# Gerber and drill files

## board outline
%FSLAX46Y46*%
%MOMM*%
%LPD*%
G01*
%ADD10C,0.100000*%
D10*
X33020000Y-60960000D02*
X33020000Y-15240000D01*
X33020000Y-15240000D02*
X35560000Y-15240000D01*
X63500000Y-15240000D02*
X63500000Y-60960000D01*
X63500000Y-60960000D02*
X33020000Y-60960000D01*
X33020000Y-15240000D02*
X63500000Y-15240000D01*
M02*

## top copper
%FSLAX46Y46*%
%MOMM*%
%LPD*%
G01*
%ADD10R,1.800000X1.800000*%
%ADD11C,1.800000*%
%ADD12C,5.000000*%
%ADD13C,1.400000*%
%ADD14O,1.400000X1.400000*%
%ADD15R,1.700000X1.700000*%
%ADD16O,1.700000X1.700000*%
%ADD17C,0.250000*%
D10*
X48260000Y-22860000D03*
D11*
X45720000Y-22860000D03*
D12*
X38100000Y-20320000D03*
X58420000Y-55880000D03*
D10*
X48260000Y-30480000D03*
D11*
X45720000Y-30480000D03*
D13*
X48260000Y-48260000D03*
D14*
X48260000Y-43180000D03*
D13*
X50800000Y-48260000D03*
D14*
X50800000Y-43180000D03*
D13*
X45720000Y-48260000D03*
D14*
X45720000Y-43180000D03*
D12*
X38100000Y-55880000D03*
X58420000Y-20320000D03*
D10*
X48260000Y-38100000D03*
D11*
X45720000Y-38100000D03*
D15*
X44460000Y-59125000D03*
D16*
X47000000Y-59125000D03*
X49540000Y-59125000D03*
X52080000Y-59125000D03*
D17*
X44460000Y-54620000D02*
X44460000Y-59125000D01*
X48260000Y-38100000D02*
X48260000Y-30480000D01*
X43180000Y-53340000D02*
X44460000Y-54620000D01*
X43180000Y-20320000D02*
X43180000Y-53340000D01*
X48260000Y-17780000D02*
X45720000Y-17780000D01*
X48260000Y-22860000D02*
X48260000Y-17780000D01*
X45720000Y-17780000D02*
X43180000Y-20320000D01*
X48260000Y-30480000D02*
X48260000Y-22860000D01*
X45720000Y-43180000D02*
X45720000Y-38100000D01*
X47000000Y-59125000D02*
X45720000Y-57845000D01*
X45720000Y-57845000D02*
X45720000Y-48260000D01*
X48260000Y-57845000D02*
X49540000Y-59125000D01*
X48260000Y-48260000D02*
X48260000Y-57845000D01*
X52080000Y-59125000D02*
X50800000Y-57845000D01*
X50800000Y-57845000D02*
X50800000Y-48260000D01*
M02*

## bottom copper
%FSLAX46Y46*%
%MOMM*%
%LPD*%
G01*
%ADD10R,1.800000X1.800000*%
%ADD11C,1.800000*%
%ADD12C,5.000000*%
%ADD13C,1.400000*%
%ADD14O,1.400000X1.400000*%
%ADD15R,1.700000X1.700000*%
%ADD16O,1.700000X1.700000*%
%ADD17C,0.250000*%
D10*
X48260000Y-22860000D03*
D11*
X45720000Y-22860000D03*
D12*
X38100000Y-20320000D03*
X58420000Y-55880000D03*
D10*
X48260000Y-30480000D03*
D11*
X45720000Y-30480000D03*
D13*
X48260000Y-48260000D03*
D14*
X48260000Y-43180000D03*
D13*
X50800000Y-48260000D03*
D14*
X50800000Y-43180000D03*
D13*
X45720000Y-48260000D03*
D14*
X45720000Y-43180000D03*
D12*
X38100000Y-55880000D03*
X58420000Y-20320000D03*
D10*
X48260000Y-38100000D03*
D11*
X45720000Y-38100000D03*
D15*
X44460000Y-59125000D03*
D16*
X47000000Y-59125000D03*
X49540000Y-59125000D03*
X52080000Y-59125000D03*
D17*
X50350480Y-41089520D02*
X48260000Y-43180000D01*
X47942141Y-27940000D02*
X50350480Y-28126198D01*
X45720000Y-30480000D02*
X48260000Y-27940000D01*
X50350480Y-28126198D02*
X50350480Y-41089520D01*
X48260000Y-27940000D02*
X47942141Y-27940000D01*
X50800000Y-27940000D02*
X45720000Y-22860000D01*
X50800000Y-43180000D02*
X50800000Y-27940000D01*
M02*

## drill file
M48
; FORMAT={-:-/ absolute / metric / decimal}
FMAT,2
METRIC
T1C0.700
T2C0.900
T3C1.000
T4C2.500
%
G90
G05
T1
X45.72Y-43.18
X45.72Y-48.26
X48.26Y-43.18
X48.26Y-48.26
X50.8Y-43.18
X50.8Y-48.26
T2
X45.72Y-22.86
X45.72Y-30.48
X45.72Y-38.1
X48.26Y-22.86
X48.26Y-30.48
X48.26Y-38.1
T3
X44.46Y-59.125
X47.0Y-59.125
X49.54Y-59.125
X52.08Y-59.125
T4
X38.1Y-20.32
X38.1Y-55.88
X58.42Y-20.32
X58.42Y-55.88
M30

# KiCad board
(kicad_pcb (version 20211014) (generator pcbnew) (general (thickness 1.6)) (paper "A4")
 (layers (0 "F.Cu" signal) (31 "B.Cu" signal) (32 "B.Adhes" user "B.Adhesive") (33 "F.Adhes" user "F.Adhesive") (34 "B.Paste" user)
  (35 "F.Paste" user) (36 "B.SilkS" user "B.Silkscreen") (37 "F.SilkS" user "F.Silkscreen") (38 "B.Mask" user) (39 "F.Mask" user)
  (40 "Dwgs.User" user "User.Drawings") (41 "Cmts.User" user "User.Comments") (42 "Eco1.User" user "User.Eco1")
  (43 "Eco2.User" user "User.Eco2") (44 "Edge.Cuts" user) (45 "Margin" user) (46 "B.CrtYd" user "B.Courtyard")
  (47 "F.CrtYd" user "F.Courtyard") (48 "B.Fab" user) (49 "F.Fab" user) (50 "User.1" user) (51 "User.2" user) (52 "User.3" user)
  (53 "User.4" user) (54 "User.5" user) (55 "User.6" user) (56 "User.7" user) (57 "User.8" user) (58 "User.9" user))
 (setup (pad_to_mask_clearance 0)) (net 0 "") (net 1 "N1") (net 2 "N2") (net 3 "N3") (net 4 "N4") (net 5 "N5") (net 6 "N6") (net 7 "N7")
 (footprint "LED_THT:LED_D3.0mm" (layer "F.Cu") (at 48.26 22.86 180)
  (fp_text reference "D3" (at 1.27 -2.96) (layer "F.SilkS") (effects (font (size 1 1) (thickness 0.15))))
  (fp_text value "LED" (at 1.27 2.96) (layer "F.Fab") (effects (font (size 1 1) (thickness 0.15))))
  (pad "1" thru_hole rect (at 0 0 180) (size 1.8 1.8) (drill 0.9) (layers *.Cu *.Mask) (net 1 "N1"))
  (pad "2" thru_hole circle (at 2.54 0 180) (size 1.8 1.8) (drill 0.9) (layers *.Cu *.Mask) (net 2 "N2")))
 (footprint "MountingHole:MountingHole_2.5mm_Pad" (layer "F.Cu") (at 38.1 20.32)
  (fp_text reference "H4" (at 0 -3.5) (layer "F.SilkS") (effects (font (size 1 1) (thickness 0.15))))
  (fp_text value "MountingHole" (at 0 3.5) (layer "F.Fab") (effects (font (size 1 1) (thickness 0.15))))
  (pad "1" thru_hole circle (at 0 0) (size 5 5) (drill 2.5) (layers *.Cu *.Mask)))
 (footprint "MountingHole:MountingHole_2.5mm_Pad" (layer "F.Cu") (at 58.42 55.88)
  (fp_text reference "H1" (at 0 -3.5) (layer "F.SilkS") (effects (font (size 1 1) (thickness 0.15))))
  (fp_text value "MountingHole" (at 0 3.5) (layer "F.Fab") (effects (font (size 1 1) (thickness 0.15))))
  (pad "1" thru_hole circle (at 0 0) (size 5 5) (drill 2.5) (layers *.Cu *.Mask)))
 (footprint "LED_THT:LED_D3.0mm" (layer "F.Cu") (at 48.26 30.48 180)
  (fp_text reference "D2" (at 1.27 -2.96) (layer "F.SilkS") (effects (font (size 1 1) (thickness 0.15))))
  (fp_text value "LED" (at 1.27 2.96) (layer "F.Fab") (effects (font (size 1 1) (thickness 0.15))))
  (pad "1" thru_hole rect (at 0 0 180) (size 1.8 1.8) (drill 0.9) (layers *.Cu *.Mask) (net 1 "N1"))
  (pad "2" thru_hole circle (at 2.54 0 180) (size 1.8 1.8) (drill 0.9) (layers *.Cu *.Mask) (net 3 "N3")))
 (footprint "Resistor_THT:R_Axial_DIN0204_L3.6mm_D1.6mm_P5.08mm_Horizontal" (layer "F.Cu") (at 48.26 48.26 90)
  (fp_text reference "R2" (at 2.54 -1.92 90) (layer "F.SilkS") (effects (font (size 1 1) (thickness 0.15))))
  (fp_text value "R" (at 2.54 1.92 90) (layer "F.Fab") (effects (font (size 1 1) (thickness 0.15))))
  (pad "1" thru_hole circle (at 0 0 90) (size 1.4 1.4) (drill 0.7) (layers *.Cu *.Mask) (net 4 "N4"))
  (pad "2" thru_hole oval (at 5.08 0 90) (size 1.4 1.4) (drill 0.7) (layers *.Cu *.Mask) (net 3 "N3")))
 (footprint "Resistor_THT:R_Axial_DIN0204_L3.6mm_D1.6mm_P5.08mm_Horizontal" (layer "F.Cu") (at 50.8 48.26 90)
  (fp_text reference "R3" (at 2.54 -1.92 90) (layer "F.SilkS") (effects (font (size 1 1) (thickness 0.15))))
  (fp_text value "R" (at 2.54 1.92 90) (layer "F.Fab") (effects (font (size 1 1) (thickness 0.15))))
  (pad "1" thru_hole circle (at 0 0 90) (size 1.4 1.4) (drill 0.7) (layers *.Cu *.Mask) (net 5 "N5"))
  (pad "2" thru_hole oval (at 5.08 0 90) (size 1.4 1.4) (drill 0.7) (layers *.Cu *.Mask) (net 2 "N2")))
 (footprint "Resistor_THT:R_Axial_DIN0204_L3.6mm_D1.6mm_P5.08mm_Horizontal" (layer "F.Cu") (at 45.72 48.26 90)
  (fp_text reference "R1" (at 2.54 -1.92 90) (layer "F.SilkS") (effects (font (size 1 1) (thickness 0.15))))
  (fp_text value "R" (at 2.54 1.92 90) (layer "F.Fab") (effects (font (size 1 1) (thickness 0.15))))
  (pad "1" thru_hole circle (at 0 0 90) (size 1.4 1.4) (drill 0.7) (layers *.Cu *.Mask) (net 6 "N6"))
  (pad "2" thru_hole oval (at 5.08 0 90) (size 1.4 1.4) (drill 0.7) (layers *.Cu *.Mask) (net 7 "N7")))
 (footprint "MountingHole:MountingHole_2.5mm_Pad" (layer "F.Cu") (at 38.1 55.88)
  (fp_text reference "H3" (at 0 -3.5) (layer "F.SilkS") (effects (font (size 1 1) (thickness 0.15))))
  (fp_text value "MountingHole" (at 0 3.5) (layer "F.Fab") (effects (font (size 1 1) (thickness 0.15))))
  (pad "1" thru_hole circle (at 0 0) (size 5 5) (drill 2.5) (layers *.Cu *.Mask)))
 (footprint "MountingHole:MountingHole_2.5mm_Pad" (layer "F.Cu") (at 58.42 20.32)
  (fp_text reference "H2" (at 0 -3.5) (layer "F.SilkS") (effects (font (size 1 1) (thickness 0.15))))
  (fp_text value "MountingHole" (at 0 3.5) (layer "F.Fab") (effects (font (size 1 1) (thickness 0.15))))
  (pad "1" thru_hole circle (at 0 0) (size 5 5) (drill 2.5) (layers *.Cu *.Mask)))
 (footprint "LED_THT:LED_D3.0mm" (layer "F.Cu") (at 48.26 38.1 180)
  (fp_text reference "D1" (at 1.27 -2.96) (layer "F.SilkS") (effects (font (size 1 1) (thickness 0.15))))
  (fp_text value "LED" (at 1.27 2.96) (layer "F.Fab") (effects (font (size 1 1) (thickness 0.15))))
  (pad "1" thru_hole rect (at 0 0 180) (size 1.8 1.8) (drill 0.9) (layers *.Cu *.Mask) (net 1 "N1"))
  (pad "2" thru_hole circle (at 2.54 0 180) (size 1.8 1.8) (drill 0.9) (layers *.Cu *.Mask) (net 7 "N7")))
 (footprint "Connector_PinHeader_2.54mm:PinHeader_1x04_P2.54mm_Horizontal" (layer "B.Cu") (at 44.46 59.125 -90)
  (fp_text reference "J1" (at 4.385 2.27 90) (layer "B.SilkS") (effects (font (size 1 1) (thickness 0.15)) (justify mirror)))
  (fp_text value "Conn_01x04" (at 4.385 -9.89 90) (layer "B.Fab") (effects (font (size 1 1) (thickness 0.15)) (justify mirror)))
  (pad "1" thru_hole rect (at 0 0 270) (size 1.7 1.7) (drill 1) (layers *.Cu *.Mask) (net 1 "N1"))
  (pad "2" thru_hole oval (at 0 -2.54 270) (size 1.7 1.7) (drill 1) (layers *.Cu *.Mask) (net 6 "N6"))
  (pad "3" thru_hole oval (at 0 -5.08 270) (size 1.7 1.7) (drill 1) (layers *.Cu *.Mask) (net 4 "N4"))
  (pad "4" thru_hole oval (at 0 -7.62 270) (size 1.7 1.7) (drill 1) (layers *.Cu *.Mask) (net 5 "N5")))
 (gr_line (start 33.02 60.96) (end 33.02 15.24) (layer "Edge.Cuts") (width 0.1))
 (gr_line (start 33.02 15.24) (end 35.56 15.24) (layer "Edge.Cuts") (width 0.1))
 (gr_line (start 63.5 15.24) (end 63.5 60.96) (layer "Edge.Cuts") (width 0.1))
 (gr_line (start 63.5 60.96) (end 33.02 60.96) (layer "Edge.Cuts") (width 0.1))
 (gr_line (start 33.02 15.24) (end 63.5 15.24) (layer "Edge.Cuts") (width 0.1))
 (segment (start 44.46 54.62) (end 44.46 59.125) (width 0.25) (layer "F.Cu") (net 1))
 (segment (start 48.26 38.1) (end 48.26 30.48) (width 0.25) (layer "F.Cu") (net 1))
 (segment (start 43.18 53.34) (end 44.46 54.62) (width 0.25) (layer "F.Cu") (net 1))
 (segment (start 43.18 20.32) (end 43.18 53.34) (width 0.25) (layer "F.Cu") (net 1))
 (segment (start 48.26 17.78) (end 45.72 17.78) (width 0.25) (layer "F.Cu") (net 1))
 (segment (start 48.26 22.86) (end 48.26 17.78) (width 0.25) (layer "F.Cu") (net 1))
 (segment (start 45.72 17.78) (end 43.18 20.32) (width 0.25) (layer "F.Cu") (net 1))
 (segment (start 48.26 30.48) (end 48.26 22.86) (width 0.25) (layer "F.Cu") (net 1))
 (segment (start 45.72 43.18) (end 45.72 38.1) (width 0.25) (layer "F.Cu") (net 7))
 (segment (start 50.35048 41.08952) (end 48.26 43.18) (width 0.25) (layer "B.Cu") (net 3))
 (segment (start 47.942141 27.94) (end 50.35048 28.126198) (width 0.25) (layer "B.Cu") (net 3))
 (segment (start 45.72 30.48) (end 48.26 27.94) (width 0.25) (layer "B.Cu") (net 3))
 (segment (start 50.35048 28.126198) (end 50.35048 41.08952) (width 0.25) (layer "B.Cu") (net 3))
 (segment (start 48.26 27.94) (end 47.942141 27.94) (width 0.25) (layer "B.Cu") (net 3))
 (segment (start 50.8 27.94) (end 45.72 22.86) (width 0.25) (layer "B.Cu") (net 2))
 (segment (start 50.8 43.18) (end 50.8 27.94) (width 0.25) (layer "B.Cu") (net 2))
 (segment (start 47 59.125) (end 45.72 57.845) (width 0.25) (layer "F.Cu") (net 6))
 (segment (start 45.72 57.845) (end 45.72 48.26) (width 0.25) (layer "F.Cu") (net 6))
 (segment (start 48.26 57.845) (end 49.54 59.125) (width 0.25) (layer "F.Cu") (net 4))
 (segment (start 48.26 48.26) (end 48.26 57.845) (width 0.25) (layer "F.Cu") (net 4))
 (segment (start 52.08 59.125) (end 50.8 57.845) (width 0.25) (layer "F.Cu") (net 5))
 (segment (start 50.8 57.845) (end 50.8 48.26) (width 0.25) (layer "F.Cu") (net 5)))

